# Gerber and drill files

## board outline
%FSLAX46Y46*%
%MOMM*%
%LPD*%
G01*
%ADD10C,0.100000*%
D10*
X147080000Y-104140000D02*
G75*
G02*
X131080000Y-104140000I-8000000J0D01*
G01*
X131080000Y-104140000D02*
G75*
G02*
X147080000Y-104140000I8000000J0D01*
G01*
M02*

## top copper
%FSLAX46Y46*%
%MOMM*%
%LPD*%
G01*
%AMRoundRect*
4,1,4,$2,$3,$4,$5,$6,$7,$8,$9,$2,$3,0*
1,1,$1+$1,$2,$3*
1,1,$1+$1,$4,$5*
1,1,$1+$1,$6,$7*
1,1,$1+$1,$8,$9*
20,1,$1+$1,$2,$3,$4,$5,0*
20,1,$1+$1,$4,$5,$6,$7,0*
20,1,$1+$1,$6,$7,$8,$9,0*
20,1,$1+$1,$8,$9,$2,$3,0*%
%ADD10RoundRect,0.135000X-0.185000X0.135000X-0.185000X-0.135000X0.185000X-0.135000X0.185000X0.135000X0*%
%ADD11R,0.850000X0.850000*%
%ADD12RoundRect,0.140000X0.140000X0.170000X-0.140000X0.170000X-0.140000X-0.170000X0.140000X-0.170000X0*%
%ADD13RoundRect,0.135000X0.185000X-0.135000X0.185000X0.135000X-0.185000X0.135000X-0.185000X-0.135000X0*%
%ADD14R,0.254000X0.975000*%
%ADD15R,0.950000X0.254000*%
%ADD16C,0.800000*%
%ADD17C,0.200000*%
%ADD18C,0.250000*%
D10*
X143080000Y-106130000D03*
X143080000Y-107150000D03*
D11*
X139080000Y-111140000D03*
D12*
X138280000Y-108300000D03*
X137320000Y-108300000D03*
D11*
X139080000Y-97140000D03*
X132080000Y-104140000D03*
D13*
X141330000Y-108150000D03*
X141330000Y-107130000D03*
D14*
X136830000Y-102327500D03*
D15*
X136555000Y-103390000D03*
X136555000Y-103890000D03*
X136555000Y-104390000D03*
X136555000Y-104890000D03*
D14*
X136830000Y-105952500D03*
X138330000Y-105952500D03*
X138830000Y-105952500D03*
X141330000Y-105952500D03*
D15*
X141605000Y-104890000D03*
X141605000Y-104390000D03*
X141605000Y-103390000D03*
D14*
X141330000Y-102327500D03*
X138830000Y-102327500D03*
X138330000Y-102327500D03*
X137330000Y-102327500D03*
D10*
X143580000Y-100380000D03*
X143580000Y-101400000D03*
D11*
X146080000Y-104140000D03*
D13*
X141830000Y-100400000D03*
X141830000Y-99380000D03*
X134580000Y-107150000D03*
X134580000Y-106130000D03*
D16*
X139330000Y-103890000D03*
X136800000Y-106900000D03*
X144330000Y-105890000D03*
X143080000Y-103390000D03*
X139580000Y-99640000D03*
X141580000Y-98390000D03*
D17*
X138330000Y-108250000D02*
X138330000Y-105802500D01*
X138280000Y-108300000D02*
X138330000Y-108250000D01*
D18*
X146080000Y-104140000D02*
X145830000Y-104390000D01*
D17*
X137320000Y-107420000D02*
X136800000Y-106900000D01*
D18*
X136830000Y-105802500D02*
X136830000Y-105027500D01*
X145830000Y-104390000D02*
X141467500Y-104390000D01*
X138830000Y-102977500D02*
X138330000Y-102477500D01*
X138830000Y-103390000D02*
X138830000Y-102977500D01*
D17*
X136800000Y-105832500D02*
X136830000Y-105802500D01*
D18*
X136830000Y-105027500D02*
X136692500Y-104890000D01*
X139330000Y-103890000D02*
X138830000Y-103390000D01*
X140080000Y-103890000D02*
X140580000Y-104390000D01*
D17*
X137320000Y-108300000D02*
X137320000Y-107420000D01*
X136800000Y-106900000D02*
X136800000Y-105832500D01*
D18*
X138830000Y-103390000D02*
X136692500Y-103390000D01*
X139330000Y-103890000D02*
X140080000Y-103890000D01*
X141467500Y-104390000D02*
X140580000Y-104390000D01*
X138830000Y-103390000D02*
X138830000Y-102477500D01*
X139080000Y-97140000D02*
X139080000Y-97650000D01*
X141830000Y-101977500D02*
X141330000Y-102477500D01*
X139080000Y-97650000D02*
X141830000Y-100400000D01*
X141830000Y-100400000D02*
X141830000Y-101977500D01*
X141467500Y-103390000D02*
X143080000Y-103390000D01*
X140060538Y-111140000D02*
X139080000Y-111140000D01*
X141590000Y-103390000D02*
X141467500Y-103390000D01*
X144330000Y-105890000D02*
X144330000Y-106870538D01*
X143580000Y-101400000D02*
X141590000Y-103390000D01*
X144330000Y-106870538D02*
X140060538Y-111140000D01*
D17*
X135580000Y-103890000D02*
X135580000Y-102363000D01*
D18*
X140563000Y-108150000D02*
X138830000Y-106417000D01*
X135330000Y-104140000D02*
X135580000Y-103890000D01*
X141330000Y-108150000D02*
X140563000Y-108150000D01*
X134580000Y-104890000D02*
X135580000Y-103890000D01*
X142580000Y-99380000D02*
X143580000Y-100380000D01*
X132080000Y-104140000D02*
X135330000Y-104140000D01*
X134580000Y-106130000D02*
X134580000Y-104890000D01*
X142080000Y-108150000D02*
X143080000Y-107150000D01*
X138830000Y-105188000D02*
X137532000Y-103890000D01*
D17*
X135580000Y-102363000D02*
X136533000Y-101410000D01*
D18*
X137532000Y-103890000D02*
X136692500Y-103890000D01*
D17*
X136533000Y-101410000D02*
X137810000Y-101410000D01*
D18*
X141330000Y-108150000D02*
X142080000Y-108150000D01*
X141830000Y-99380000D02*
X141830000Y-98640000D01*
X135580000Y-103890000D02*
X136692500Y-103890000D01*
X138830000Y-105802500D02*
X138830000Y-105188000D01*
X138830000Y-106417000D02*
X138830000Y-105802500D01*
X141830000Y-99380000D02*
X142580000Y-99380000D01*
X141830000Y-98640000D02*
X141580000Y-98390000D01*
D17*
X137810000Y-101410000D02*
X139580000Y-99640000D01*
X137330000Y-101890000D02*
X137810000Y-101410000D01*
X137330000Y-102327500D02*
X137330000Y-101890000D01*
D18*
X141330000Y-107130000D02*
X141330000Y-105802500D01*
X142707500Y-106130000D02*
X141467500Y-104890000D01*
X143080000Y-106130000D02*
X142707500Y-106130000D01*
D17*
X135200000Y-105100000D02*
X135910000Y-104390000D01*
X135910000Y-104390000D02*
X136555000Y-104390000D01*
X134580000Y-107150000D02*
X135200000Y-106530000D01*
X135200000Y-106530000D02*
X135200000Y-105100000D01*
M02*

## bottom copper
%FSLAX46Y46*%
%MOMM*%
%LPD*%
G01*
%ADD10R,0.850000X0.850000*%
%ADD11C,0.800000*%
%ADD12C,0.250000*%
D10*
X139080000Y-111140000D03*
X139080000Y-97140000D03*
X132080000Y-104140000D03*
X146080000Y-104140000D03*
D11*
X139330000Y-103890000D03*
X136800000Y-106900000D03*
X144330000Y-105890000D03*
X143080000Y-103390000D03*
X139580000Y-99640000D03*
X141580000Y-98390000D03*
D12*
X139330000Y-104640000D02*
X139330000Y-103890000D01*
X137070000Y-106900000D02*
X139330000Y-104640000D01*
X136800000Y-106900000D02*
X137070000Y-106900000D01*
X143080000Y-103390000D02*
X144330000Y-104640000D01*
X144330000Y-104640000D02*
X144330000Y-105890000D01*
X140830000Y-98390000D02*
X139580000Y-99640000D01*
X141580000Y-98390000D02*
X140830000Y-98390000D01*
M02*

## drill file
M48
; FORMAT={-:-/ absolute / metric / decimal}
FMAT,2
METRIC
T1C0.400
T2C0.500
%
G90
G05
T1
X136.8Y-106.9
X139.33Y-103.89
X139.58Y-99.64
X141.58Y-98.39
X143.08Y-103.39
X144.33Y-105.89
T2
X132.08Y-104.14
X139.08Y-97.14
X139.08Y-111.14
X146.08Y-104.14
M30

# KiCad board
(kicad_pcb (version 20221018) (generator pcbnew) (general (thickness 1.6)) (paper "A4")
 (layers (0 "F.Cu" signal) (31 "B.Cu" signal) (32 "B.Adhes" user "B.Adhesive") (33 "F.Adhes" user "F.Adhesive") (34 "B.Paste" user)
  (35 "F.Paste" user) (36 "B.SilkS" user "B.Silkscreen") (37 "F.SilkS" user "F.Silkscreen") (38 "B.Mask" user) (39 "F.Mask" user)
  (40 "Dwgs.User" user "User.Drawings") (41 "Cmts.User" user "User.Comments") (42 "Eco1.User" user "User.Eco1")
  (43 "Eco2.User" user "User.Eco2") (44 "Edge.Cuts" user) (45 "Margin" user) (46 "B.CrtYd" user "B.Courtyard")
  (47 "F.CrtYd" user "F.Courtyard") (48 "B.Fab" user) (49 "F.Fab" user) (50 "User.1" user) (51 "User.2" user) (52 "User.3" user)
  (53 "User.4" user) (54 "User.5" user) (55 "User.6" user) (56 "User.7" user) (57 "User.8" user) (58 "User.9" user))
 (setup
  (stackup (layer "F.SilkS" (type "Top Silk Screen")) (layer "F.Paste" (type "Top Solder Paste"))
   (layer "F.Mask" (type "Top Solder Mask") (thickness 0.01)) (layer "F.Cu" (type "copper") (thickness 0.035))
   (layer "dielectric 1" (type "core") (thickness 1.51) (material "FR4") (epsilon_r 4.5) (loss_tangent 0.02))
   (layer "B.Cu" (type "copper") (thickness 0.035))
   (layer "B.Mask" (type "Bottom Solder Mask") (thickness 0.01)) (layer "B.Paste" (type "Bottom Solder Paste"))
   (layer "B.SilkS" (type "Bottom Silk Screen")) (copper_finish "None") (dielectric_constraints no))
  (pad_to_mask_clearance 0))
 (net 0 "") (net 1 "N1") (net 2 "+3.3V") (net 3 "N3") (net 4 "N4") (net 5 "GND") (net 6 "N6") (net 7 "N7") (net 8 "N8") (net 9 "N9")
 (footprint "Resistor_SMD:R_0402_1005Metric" (layer "F.Cu") (at 143.08 106.64 -90)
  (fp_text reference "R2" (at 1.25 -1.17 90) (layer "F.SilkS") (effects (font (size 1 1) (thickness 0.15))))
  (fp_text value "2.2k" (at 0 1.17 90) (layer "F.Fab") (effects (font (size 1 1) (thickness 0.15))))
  (pad "1" smd roundrect (at -0.51 0 270) (size 0.54 0.64) (layers "F.Cu" "F.Paste" "F.Mask") (roundrect_rratio 0.25) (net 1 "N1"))
  (pad "2" smd roundrect (at 0.51 0 270) (size 0.54 0.64) (layers "F.Cu" "F.Paste" "F.Mask") (roundrect_rratio 0.25) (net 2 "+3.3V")))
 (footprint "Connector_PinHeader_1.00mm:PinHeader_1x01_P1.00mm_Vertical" (layer "F.Cu") (at 139.08 111.14 180)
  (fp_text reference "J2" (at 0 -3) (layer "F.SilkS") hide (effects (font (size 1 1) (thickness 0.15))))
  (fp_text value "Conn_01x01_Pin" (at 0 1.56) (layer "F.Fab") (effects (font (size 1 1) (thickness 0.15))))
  (pad "1" thru_hole rect (at 0 0 180) (size 0.85 0.85) (drill 0.5) (layers "*.Cu" "*.Mask") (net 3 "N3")))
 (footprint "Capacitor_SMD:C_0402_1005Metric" (layer "F.Cu") (at 137.8 108.3 180)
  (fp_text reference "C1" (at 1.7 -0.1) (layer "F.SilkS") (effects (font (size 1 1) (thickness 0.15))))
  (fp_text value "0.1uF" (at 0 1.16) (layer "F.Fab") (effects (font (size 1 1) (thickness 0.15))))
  (pad "1" smd roundrect (at -0.48 0 180) (size 0.56 0.62) (layers "F.Cu" "F.Paste" "F.Mask") (roundrect_rratio 0.25) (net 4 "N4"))
  (pad "2" smd roundrect (at 0.48 0 180) (size 0.56 0.62) (layers "F.Cu" "F.Paste" "F.Mask") (roundrect_rratio 0.25) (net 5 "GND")))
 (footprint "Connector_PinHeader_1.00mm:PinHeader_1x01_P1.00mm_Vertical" (layer "F.Cu") (at 139.08 97.14)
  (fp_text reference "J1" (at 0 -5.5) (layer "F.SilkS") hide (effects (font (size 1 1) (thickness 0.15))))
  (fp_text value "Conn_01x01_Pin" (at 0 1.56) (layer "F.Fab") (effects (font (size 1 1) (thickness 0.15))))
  (pad "1" thru_hole rect (at 0 0) (size 0.85 0.85) (drill 0.5) (layers "*.Cu" "*.Mask") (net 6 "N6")))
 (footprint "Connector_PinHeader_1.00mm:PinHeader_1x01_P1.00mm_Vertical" (layer "F.Cu") (at 132.08 104.14 90)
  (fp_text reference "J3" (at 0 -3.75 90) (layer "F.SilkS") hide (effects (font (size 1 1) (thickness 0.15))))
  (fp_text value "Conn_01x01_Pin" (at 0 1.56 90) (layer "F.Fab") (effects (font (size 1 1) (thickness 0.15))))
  (pad "1" thru_hole rect (at 0 0 90) (size 0.85 0.85) (drill 0.5) (layers "*.Cu" "*.Mask") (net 2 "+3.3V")))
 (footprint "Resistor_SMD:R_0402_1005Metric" (layer "F.Cu") (at 141.33 107.64 90)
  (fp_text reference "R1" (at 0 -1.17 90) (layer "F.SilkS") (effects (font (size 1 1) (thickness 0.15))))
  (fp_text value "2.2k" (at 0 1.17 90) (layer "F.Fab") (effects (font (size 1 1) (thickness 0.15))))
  (pad "1" smd roundrect (at -0.51 0 90) (size 0.54 0.64) (layers "F.Cu" "F.Paste" "F.Mask") (roundrect_rratio 0.25) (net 2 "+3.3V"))
  (pad "2" smd roundrect (at 0.51 0 90) (size 0.54 0.64) (layers "F.Cu" "F.Paste" "F.Mask") (roundrect_rratio 0.25) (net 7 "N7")))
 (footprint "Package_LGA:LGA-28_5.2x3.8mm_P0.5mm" (layer "F.Cu") (at 139.08 104.14)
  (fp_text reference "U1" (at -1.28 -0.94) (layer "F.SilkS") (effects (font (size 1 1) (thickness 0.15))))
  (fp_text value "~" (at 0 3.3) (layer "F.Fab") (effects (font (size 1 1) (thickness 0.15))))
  (pad "1" smd rect (at -2.25 -1.8125) (size 0.254 0.975) (layers "F.Cu" "F.Paste" "F.Mask") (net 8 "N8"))
  (pad "2" smd rect (at -2.525 -0.75 90) (size 0.254 0.95) (layers "F.Cu" "F.Paste" "F.Mask") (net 5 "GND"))
  (pad "3" smd rect (at -2.525 -0.25 90) (size 0.254 0.95) (layers "F.Cu" "F.Paste" "F.Mask") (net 2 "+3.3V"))
  (pad "4" smd rect (at -2.525 0.25 90) (size 0.254 0.95) (layers "F.Cu" "F.Paste" "F.Mask") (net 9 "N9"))
  (pad "5" smd rect (at -2.525 0.75 90) (size 0.254 0.95) (layers "F.Cu" "F.Paste" "F.Mask") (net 5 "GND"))
  (pad "6" smd rect (at -2.25 1.8125) (size 0.254 0.975) (layers "F.Cu" "F.Paste" "F.Mask") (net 5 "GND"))
  (pad "9" smd rect (at -0.75 1.8125) (size 0.254 0.975) (layers "F.Cu" "F.Paste" "F.Mask") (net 4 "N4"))
  (pad "10" smd rect (at -0.25 1.8125) (size 0.254 0.975) (layers "F.Cu" "F.Paste" "F.Mask") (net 2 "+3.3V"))
  (pad "15" smd rect (at 2.25 1.8125) (size 0.254 0.975) (layers "F.Cu" "F.Paste" "F.Mask") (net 7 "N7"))
  (pad "16" smd rect (at 2.525 0.75 90) (size 0.254 0.95) (layers "F.Cu" "F.Paste" "F.Mask") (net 1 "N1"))
  (pad "17" smd rect (at 2.525 0.25 90) (size 0.254 0.95) (layers "F.Cu" "F.Paste" "F.Mask") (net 5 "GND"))
  (pad "19" smd rect (at 2.525 -0.75 90) (size 0.254 0.95) (layers "F.Cu" "F.Paste" "F.Mask") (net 3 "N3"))
  (pad "20" smd rect (at 2.25 -1.8125) (size 0.254 0.975) (layers "F.Cu" "F.Paste" "F.Mask") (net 6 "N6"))
  (pad "25" smd rect (at -0.25 -1.8125) (size 0.254 0.975) (layers "F.Cu" "F.Paste" "F.Mask") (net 5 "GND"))
  (pad "26" smd rect (at -0.75 -1.8125) (size 0.254 0.975) (layers "F.Cu" "F.Paste" "F.Mask") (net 5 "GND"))
  (pad "28" smd rect (at -1.75 -1.8125) (size 0.254 0.975) (layers "F.Cu" "F.Paste" "F.Mask") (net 2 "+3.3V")))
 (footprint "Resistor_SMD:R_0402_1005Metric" (layer "F.Cu") (at 143.58 100.89 -90)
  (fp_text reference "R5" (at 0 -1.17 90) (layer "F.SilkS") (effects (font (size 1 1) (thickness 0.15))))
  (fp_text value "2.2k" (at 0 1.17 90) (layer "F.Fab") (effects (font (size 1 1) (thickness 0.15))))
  (pad "1" smd roundrect (at -0.51 0 270) (size 0.54 0.64) (layers "F.Cu" "F.Paste" "F.Mask") (roundrect_rratio 0.25) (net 2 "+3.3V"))
  (pad "2" smd roundrect (at 0.51 0 270) (size 0.54 0.64) (layers "F.Cu" "F.Paste" "F.Mask") (roundrect_rratio 0.25) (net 3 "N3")))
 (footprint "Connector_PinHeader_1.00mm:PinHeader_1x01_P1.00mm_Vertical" (layer "F.Cu") (at 146.08 104.14 -90)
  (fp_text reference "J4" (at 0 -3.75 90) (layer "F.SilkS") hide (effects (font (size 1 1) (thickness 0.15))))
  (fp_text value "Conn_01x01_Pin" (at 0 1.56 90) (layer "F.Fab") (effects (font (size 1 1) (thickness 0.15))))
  (pad "1" thru_hole rect (at 0 0 270) (size 0.85 0.85) (drill 0.5) (layers "*.Cu" "*.Mask") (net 5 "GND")))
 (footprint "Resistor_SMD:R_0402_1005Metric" (layer "F.Cu") (at 141.83 99.89 90)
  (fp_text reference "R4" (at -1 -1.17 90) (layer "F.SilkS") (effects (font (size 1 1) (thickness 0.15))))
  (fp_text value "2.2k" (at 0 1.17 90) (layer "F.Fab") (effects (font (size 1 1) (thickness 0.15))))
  (pad "1" smd roundrect (at -0.51 0 90) (size 0.54 0.64) (layers "F.Cu" "F.Paste" "F.Mask") (roundrect_rratio 0.25) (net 6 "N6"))
  (pad "2" smd roundrect (at 0.51 0 90) (size 0.54 0.64) (layers "F.Cu" "F.Paste" "F.Mask") (roundrect_rratio 0.25) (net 2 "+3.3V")))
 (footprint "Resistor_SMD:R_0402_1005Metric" (layer "F.Cu") (at 134.58 106.64 90)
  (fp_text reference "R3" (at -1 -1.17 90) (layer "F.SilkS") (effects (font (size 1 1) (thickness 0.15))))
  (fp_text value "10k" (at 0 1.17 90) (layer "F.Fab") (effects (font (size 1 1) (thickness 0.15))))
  (pad "1" smd roundrect (at -0.51 0 90) (size 0.54 0.64) (layers "F.Cu" "F.Paste" "F.Mask") (roundrect_rratio 0.25) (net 9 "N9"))
  (pad "2" smd roundrect (at 0.51 0 90) (size 0.54 0.64) (layers "F.Cu" "F.Paste" "F.Mask") (roundrect_rratio 0.25) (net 2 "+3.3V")))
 (gr_circle (center 139.08 104.14) (end 147.08 104.14) (stroke (width 0.1) (type default)) (fill none) (layer "Edge.Cuts"))
 (segment (start 138.33 108.25) (end 138.33 105.8025) (width 0.2) (layer "F.Cu") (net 4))
 (segment (start 138.28 108.3) (end 138.33 108.25) (width 0.2) (layer "F.Cu") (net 4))
 (segment (start 146.08 104.14) (end 145.83 104.39) (width 0.25) (layer "F.Cu") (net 5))
 (segment (start 137.32 107.42) (end 136.8 106.9) (width 0.2) (layer "F.Cu") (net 5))
 (segment (start 136.83 105.8025) (end 136.83 105.0275) (width 0.25) (layer "F.Cu") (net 5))
 (segment (start 145.83 104.39) (end 141.4675 104.39) (width 0.25) (layer "F.Cu") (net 5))
 (segment (start 138.83 102.9775) (end 138.33 102.4775) (width 0.25) (layer "F.Cu") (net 5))
 (segment (start 138.83 103.39) (end 138.83 102.9775) (width 0.25) (layer "F.Cu") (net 5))
 (segment (start 136.8 105.8325) (end 136.83 105.8025) (width 0.2) (layer "F.Cu") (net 5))
 (segment (start 136.83 105.0275) (end 136.6925 104.89) (width 0.25) (layer "F.Cu") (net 5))
 (segment (start 139.33 103.89) (end 138.83 103.39) (width 0.25) (layer "F.Cu") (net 5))
 (segment (start 140.08 103.89) (end 140.58 104.39) (width 0.25) (layer "F.Cu") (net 5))
 (segment (start 137.32 108.3) (end 137.32 107.42) (width 0.2) (layer "F.Cu") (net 5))
 (segment (start 136.8 106.9) (end 136.8 105.8325) (width 0.2) (layer "F.Cu") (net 5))
 (segment (start 138.83 103.39) (end 136.6925 103.39) (width 0.25) (layer "F.Cu") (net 5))
 (segment (start 139.33 103.89) (end 140.08 103.89) (width 0.25) (layer "F.Cu") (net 5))
 (segment (start 141.4675 104.39) (end 140.58 104.39) (width 0.25) (layer "F.Cu") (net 5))
 (segment (start 138.83 103.39) (end 138.83 102.4775) (width 0.25) (layer "F.Cu") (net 5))
 (via (at 139.33 103.89) (size 0.8) (drill 0.4) (layers "F.Cu" "B.Cu") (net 5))
 (via (at 136.8 106.9) (size 0.8) (drill 0.4) (layers "F.Cu" "B.Cu") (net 5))
 (segment (start 139.33 104.64) (end 139.33 103.89) (width 0.25) (layer "B.Cu") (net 5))
 (segment (start 137.07 106.9) (end 139.33 104.64) (width 0.25) (layer "B.Cu") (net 5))
 (segment (start 136.8 106.9) (end 137.07 106.9) (width 0.25) (layer "B.Cu") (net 5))
 (segment (start 139.08 97.14) (end 139.08 97.65) (width 0.25) (layer "F.Cu") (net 6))
 (segment (start 141.83 101.9775) (end 141.33 102.4775) (width 0.25) (layer "F.Cu") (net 6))
 (segment (start 139.08 97.65) (end 141.83 100.4) (width 0.25) (layer "F.Cu") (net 6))
 (segment (start 141.83 100.4) (end 141.83 101.9775) (width 0.25) (layer "F.Cu") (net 6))
 (segment (start 141.4675 103.39) (end 143.08 103.39) (width 0.25) (layer "F.Cu") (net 3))
 (segment (start 140.060538 111.14) (end 139.08 111.14) (width 0.25) (layer "F.Cu") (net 3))
 (segment (start 141.59 103.39) (end 141.4675 103.39) (width 0.25) (layer "F.Cu") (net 3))
 (segment (start 144.33 105.89) (end 144.33 106.870538) (width 0.25) (layer "F.Cu") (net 3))
 (segment (start 143.58 101.4) (end 141.59 103.39) (width 0.25) (layer "F.Cu") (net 3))
 (segment (start 144.33 106.870538) (end 140.060538 111.14) (width 0.25) (layer "F.Cu") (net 3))
 (via (at 144.33 105.89) (size 0.8) (drill 0.4) (layers "F.Cu" "B.Cu") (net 3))
 (via (at 143.08 103.39) (size 0.8) (drill 0.4) (layers "F.Cu" "B.Cu") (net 3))
 (segment (start 143.08 103.39) (end 144.33 104.64) (width 0.25) (layer "B.Cu") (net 3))
 (segment (start 144.33 104.64) (end 144.33 105.89) (width 0.25) (layer "B.Cu") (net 3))
 (segment (start 135.58 103.89) (end 135.58 102.363) (width 0.2) (layer "F.Cu") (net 2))
 (segment (start 140.563 108.15) (end 138.83 106.417) (width 0.25) (layer "F.Cu") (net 2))
 (segment (start 135.33 104.14) (end 135.58 103.89) (width 0.25) (layer "F.Cu") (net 2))
 (segment (start 141.33 108.15) (end 140.563 108.15) (width 0.25) (layer "F.Cu") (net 2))
 (segment (start 134.58 104.89) (end 135.58 103.89) (width 0.25) (layer "F.Cu") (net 2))
 (segment (start 142.58 99.38) (end 143.58 100.38) (width 0.25) (layer "F.Cu") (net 2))
 (segment (start 132.08 104.14) (end 135.33 104.14) (width 0.25) (layer "F.Cu") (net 2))
 (segment (start 134.58 106.13) (end 134.58 104.89) (width 0.25) (layer "F.Cu") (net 2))
 (segment (start 142.08 108.15) (end 143.08 107.15) (width 0.25) (layer "F.Cu") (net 2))
 (segment (start 138.83 105.188) (end 137.532 103.89) (width 0.25) (layer "F.Cu") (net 2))
 (segment (start 135.58 102.363) (end 136.533 101.41) (width 0.2) (layer "F.Cu") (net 2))
 (segment (start 137.532 103.89) (end 136.6925 103.89) (width 0.25) (layer "F.Cu") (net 2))
 (segment (start 136.533 101.41) (end 137.81 101.41) (width 0.2) (layer "F.Cu") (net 2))
 (segment (start 141.33 108.15) (end 142.08 108.15) (width 0.25) (layer "F.Cu") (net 2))
 (segment (start 141.83 99.38) (end 141.83 98.64) (width 0.25) (layer "F.Cu") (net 2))
 (segment (start 135.58 103.89) (end 136.6925 103.89) (width 0.25) (layer "F.Cu") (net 2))
 (segment (start 138.83 105.8025) (end 138.83 105.188) (width 0.25) (layer "F.Cu") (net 2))
 (segment (start 138.83 106.417) (end 138.83 105.8025) (width 0.25) (layer "F.Cu") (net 2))
 (segment (start 141.83 99.38) (end 142.58 99.38) (width 0.25) (layer "F.Cu") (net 2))
 (segment (start 141.83 98.64) (end 141.58 98.39) (width 0.25) (layer "F.Cu") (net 2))
 (segment (start 137.81 101.41) (end 139.58 99.64) (width 0.2) (layer "F.Cu") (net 2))
 (segment (start 137.33 101.89) (end 137.81 101.41) (width 0.2) (layer "F.Cu") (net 2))
 (segment (start 137.33 102.3275) (end 137.33 101.89) (width 0.2) (layer "F.Cu") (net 2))
 (via (at 139.58 99.64) (size 0.8) (drill 0.4) (layers "F.Cu" "B.Cu") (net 2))
 (via (at 141.58 98.39) (size 0.8) (drill 0.4) (layers "F.Cu" "B.Cu") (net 2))
 (segment (start 140.83 98.39) (end 139.58 99.64) (width 0.25) (layer "B.Cu") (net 2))
 (segment (start 141.58 98.39) (end 140.83 98.39) (width 0.25) (layer "B.Cu") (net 2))
 (segment (start 141.33 107.13) (end 141.33 105.8025) (width 0.25) (layer "F.Cu") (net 7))
 (segment (start 142.7075 106.13) (end 141.4675 104.89) (width 0.25) (layer "F.Cu") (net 1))
 (segment (start 143.08 106.13) (end 142.7075 106.13) (width 0.25) (layer "F.Cu") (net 1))
 (segment (start 135.2 105.1) (end 135.91 104.39) (width 0.2) (layer "F.Cu") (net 9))
 (segment (start 135.91 104.39) (end 136.555 104.39) (width 0.2) (layer "F.Cu") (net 9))
 (segment (start 134.58 107.15) (end 135.2 106.53) (width 0.2) (layer "F.Cu") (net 9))
 (segment (start 135.2 106.53) (end 135.2 105.1) (width 0.2) (layer "F.Cu") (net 9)))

